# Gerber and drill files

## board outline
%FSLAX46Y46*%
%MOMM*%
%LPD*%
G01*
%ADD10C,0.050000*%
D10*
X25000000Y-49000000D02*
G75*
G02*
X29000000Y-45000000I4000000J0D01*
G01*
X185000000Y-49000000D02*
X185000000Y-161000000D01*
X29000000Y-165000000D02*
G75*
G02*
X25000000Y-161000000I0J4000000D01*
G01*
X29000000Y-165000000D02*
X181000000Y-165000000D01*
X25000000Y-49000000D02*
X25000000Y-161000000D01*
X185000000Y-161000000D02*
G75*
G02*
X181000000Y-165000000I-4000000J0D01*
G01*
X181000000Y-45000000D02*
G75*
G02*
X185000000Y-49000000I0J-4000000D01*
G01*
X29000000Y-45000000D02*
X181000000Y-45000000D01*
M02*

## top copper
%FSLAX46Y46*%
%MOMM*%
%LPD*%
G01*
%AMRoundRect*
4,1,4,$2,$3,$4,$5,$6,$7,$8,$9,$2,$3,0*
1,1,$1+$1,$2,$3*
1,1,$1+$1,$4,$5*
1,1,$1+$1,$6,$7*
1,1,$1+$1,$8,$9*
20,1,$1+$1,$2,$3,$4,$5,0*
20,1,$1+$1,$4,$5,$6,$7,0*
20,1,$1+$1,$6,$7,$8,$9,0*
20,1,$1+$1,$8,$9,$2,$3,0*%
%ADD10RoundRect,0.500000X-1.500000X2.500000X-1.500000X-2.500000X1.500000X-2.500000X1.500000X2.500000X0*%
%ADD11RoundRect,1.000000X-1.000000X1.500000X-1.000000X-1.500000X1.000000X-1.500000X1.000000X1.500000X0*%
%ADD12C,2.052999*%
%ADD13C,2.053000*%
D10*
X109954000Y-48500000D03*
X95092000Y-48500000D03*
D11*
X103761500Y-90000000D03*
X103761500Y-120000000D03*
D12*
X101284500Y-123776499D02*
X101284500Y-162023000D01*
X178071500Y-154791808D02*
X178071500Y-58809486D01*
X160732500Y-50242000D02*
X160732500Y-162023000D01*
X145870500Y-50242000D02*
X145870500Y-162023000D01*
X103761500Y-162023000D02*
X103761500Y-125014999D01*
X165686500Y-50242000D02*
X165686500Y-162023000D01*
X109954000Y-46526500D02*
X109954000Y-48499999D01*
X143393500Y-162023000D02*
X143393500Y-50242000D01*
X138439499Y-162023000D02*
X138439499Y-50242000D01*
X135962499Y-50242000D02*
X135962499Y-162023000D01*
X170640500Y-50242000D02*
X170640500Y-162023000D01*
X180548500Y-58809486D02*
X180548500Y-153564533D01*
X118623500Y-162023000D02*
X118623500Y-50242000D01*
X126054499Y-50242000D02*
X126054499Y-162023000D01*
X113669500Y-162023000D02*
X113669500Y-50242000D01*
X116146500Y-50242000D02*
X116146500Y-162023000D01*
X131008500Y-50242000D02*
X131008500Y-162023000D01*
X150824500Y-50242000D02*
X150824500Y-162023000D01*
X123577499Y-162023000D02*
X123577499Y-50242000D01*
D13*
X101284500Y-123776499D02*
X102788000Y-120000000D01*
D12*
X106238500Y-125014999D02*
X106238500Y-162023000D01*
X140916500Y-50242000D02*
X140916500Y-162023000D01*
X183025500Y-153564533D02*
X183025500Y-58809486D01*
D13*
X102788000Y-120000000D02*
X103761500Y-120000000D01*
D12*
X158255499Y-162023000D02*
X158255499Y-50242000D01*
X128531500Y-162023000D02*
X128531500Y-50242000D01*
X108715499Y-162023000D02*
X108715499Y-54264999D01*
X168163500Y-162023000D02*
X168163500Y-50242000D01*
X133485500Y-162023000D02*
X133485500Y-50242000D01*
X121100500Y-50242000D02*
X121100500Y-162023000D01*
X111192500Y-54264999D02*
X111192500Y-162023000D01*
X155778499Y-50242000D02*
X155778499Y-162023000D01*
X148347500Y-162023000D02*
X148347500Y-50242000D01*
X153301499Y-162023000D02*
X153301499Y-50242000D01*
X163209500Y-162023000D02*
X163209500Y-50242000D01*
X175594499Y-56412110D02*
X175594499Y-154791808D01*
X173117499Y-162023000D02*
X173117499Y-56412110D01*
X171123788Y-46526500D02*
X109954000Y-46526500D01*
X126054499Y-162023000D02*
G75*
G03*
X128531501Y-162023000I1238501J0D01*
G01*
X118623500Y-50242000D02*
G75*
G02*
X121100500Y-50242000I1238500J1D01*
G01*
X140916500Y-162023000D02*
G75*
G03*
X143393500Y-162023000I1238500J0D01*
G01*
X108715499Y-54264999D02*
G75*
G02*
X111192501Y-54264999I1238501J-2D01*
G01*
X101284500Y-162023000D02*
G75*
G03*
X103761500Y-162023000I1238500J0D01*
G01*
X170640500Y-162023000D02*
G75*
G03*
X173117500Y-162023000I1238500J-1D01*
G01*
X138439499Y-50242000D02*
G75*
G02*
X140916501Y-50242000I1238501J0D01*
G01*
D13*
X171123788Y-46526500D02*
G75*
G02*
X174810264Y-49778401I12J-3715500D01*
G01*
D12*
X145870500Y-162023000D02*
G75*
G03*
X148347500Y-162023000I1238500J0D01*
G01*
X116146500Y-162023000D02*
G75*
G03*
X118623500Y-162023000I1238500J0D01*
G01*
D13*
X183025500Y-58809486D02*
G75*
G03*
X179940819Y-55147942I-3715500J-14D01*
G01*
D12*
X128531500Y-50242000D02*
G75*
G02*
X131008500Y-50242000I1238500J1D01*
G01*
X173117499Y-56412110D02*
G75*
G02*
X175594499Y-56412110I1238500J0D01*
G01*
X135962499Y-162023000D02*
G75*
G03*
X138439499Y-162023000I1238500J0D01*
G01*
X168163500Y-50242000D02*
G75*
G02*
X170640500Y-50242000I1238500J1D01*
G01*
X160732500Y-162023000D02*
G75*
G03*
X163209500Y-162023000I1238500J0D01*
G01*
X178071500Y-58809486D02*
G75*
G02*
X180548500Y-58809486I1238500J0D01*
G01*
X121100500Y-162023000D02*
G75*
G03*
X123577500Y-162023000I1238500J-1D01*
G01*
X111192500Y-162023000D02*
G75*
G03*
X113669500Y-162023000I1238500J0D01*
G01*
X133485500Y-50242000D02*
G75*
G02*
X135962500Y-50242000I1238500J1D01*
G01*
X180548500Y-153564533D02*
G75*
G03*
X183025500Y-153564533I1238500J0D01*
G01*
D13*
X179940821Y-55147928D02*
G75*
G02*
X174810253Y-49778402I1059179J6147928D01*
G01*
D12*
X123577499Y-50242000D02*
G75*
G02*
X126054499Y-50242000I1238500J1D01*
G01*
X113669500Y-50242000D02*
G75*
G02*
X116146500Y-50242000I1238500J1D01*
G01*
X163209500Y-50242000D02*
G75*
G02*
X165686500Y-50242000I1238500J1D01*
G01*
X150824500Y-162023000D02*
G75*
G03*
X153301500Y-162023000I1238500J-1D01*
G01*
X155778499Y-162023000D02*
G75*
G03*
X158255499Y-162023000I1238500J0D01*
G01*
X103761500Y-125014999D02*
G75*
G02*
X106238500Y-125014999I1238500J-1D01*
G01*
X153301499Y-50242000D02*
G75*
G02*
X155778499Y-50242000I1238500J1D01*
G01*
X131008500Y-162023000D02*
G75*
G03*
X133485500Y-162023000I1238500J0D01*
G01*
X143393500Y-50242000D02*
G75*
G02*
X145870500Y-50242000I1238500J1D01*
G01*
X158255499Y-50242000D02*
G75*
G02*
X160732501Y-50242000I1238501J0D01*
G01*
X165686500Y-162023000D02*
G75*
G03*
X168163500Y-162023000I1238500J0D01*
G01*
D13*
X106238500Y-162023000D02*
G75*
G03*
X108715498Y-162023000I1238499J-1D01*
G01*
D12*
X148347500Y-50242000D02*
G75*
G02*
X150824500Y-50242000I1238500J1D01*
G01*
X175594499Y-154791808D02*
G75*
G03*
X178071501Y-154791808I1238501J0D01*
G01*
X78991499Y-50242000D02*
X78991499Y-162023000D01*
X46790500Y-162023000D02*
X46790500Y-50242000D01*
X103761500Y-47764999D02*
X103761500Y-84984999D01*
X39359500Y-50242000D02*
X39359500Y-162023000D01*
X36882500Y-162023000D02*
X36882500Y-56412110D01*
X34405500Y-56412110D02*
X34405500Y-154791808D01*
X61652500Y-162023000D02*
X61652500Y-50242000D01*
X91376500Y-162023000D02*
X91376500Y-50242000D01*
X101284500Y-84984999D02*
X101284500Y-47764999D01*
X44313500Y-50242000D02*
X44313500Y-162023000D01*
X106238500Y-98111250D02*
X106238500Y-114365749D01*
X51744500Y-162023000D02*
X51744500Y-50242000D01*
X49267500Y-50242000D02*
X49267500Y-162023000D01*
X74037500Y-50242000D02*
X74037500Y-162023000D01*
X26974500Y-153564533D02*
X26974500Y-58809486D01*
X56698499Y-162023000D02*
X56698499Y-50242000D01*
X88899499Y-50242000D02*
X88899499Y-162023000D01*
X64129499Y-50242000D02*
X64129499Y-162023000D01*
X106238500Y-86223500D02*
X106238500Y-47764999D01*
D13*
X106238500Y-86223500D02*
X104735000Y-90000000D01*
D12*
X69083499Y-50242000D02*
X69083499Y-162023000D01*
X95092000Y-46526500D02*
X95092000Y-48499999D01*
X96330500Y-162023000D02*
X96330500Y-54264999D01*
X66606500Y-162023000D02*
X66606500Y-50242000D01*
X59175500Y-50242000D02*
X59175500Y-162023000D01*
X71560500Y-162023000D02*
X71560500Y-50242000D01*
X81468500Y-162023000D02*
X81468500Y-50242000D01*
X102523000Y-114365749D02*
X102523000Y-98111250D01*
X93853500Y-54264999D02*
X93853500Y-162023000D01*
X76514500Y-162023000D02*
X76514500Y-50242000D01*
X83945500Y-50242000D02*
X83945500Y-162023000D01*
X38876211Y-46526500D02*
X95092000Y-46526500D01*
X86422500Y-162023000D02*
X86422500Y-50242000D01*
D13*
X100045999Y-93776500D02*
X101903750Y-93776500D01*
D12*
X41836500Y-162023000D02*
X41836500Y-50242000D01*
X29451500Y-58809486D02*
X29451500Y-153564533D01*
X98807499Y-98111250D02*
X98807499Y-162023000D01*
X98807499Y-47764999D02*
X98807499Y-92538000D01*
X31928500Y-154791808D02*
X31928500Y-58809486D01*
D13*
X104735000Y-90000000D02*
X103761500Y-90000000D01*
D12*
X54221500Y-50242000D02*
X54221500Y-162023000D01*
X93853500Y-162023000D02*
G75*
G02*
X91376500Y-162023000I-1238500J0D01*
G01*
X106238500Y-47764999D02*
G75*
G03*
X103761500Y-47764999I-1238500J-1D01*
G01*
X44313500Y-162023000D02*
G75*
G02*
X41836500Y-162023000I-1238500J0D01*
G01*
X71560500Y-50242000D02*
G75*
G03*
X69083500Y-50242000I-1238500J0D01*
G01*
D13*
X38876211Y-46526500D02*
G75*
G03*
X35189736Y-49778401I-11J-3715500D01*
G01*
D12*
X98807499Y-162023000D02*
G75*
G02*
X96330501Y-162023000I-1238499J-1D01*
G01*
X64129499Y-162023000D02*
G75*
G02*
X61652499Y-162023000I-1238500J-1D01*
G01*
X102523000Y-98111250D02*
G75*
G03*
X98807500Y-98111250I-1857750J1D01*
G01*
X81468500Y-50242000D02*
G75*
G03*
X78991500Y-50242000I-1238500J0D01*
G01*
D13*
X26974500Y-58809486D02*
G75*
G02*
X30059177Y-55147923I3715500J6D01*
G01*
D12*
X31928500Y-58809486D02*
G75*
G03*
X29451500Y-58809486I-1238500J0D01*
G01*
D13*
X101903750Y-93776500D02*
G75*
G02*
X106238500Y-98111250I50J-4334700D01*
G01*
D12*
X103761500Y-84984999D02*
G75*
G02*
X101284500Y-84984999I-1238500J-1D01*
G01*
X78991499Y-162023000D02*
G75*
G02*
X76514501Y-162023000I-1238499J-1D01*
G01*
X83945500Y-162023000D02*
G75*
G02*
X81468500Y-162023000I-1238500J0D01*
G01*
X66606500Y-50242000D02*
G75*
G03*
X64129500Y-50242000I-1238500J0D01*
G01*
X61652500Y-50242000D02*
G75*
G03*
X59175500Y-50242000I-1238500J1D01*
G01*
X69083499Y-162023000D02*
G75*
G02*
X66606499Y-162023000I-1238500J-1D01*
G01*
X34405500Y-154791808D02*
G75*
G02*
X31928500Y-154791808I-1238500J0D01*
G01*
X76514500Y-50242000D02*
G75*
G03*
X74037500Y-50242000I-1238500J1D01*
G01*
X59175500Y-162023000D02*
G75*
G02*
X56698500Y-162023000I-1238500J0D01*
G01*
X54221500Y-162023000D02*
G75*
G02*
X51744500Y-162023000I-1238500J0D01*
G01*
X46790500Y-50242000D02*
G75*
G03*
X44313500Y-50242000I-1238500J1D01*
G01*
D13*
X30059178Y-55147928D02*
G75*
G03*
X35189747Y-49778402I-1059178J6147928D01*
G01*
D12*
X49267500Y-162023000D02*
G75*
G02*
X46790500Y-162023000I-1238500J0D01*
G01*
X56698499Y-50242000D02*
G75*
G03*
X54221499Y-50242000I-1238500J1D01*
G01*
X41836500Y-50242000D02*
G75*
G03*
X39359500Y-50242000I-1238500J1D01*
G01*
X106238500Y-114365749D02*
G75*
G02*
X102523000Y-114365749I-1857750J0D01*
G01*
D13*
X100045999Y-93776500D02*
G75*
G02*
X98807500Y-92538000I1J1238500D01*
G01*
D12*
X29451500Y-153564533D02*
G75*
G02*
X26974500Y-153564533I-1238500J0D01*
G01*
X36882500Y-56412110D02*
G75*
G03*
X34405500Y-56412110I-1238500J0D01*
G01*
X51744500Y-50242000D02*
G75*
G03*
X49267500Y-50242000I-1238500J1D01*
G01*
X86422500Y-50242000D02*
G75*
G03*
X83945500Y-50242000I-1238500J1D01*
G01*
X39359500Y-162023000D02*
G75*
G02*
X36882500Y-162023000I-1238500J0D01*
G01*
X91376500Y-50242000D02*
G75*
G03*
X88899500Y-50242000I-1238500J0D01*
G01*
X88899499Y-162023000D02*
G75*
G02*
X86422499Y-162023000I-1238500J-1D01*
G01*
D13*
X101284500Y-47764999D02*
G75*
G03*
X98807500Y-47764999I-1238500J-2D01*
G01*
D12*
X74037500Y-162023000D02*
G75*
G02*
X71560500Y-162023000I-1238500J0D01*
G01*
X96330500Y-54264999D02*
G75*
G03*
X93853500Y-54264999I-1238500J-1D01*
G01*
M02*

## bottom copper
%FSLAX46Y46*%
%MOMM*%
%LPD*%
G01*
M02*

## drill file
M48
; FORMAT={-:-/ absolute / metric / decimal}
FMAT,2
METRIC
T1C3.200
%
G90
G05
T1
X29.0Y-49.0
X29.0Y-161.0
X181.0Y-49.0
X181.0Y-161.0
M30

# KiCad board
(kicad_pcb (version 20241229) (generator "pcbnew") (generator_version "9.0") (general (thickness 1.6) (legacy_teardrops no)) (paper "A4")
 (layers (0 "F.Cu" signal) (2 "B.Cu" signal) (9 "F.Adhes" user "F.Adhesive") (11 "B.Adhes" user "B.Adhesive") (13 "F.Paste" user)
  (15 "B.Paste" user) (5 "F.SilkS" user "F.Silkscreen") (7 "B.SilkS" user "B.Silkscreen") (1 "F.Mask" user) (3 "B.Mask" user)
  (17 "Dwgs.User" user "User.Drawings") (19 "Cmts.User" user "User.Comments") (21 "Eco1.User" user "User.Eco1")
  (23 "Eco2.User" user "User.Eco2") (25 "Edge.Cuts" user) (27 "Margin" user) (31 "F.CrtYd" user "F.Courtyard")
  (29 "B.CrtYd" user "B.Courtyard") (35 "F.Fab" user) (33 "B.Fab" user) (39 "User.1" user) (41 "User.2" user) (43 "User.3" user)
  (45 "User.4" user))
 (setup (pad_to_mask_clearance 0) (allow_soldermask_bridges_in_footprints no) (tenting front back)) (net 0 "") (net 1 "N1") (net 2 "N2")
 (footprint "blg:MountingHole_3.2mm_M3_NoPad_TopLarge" (layer "F.Cu") (at 181 49)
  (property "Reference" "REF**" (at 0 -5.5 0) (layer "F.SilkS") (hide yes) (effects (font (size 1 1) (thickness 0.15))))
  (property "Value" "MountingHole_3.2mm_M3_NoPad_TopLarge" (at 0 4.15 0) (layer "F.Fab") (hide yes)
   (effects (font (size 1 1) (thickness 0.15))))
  (pad "" np_thru_hole circle (at 0 0) (size 7.6 7.6) (drill 3.2) (layers) (zone_connect 2)))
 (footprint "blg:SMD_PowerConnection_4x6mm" (layer "F.Cu") (at 109.954 48.5 -90)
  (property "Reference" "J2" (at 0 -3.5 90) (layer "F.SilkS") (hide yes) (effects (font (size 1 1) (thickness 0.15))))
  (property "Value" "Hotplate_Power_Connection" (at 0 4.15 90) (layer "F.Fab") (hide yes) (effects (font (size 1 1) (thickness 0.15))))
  (pad "1" smd roundrect (at 0 0 270) (size 6 4) (layers "F.Cu" "F.Mask" "F.Paste") (roundrect_rratio 0.125) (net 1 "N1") (zone_connect 2)))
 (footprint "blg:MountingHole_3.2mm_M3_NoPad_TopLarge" (layer "F.Cu") (at 29 161)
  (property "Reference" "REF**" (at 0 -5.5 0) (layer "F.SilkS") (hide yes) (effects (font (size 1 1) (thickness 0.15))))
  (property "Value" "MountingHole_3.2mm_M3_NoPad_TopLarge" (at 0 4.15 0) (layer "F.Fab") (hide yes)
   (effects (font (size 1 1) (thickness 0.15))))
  (pad "" np_thru_hole circle (at 0 0) (size 7.6 7.6) (drill 3.2) (layers) (zone_connect 2)))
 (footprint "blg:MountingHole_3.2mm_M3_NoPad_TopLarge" (layer "F.Cu") (at 181 161)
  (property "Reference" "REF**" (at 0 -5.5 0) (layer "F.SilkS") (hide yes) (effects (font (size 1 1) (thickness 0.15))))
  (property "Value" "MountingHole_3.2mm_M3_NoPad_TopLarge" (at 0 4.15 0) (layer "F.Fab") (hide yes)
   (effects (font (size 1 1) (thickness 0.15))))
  (pad "" np_thru_hole circle (at 0 0) (size 7.6 7.6) (drill 3.2) (layers) (zone_connect 2)))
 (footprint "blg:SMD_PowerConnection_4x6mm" (layer "F.Cu") (at 95.092 48.5 -90)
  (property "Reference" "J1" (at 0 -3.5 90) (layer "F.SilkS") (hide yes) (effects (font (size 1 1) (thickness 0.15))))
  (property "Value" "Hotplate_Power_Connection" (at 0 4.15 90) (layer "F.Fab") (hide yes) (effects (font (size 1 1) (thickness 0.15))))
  (pad "1" smd roundrect (at 0 0 270) (size 6 4) (layers "F.Cu" "F.Mask" "F.Paste") (roundrect_rratio 0.125) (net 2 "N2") (zone_connect 2)))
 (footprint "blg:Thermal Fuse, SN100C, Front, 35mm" (layer "F.Cu") (at 103.7615 105 -90)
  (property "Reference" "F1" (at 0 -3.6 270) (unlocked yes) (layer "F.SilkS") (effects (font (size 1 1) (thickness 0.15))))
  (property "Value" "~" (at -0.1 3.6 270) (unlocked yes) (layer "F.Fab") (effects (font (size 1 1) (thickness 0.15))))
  (pad "1" smd roundrect (at -15 0 270) (size 5 4) (layers "F.Cu" "F.Mask") (roundrect_rratio 0.25) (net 2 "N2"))
  (pad "2" smd roundrect (at 15 0 270) (size 5 4) (layers "F.Cu" "F.Mask") (roundrect_rratio 0.25) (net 1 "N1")))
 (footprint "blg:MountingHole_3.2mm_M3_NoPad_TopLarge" (layer "F.Cu") (at 29 49)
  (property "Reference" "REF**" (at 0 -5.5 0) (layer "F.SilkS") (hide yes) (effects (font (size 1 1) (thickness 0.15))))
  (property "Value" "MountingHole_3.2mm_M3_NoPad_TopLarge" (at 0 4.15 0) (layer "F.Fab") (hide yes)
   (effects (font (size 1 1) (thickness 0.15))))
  (pad "" np_thru_hole circle (at 0 0) (size 7.6 7.6) (drill 3.2) (layers) (zone_connect 2)))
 (gr_arc (start 25 49) (mid 26.171573 46.171573) (end 29 45) (stroke (width 0.05) (type solid)) (layer "Edge.Cuts"))
 (gr_line (start 185 49) (end 185 161) (stroke (width 0.05) (type default)) (layer "Edge.Cuts"))
 (gr_arc (start 29 165) (mid 26.171573 163.828427) (end 25 161) (stroke (width 0.05) (type solid)) (layer "Edge.Cuts"))
 (gr_line (start 29 165) (end 181 165) (stroke (width 0.05) (type default)) (layer "Edge.Cuts"))
 (gr_line (start 25 49) (end 25 161) (stroke (width 0.05) (type default)) (layer "Edge.Cuts"))
 (gr_arc (start 185 161) (mid 183.828427 163.828427) (end 181 165) (stroke (width 0.05) (type solid)) (layer "Edge.Cuts"))
 (gr_arc (start 181 45) (mid 183.828427 46.171573) (end 185 49) (stroke (width 0.05) (type solid)) (layer "Edge.Cuts"))
 (gr_line (start 29 45) (end 181 45) (stroke (width 0.05) (type default)) (layer "Edge.Cuts"))
 (segment (start 101.2845 123.776499) (end 101.2845 162.023) (width 2.052999) (layer "F.Cu") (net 1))
 (segment (start 178.0715 154.791808) (end 178.0715 58.809486) (width 2.052999) (layer "F.Cu") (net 1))
 (segment (start 160.7325 50.242) (end 160.7325 162.023) (width 2.052999) (layer "F.Cu") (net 1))
 (segment (start 145.8705 50.242) (end 145.8705 162.023) (width 2.052999) (layer "F.Cu") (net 1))
 (segment (start 103.7615 162.023) (end 103.7615 125.014999) (width 2.052999) (layer "F.Cu") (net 1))
 (segment (start 165.6865 50.242) (end 165.6865 162.023) (width 2.052999) (layer "F.Cu") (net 1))
 (segment (start 109.954 46.5265) (end 109.954 48.499999) (width 2.052999) (layer "F.Cu") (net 1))
 (segment (start 143.3935 162.023) (end 143.3935 50.242) (width 2.052999) (layer "F.Cu") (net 1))
 (segment (start 138.439499 162.023) (end 138.439499 50.242) (width 2.052999) (layer "F.Cu") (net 1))
 (segment (start 135.962499 50.242) (end 135.962499 162.023) (width 2.052999) (layer "F.Cu") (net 1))
 (segment (start 170.6405 50.242) (end 170.6405 162.023) (width 2.052999) (layer "F.Cu") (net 1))
 (segment (start 180.5485 58.809486) (end 180.5485 153.564533) (width 2.052999) (layer "F.Cu") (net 1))
 (segment (start 118.6235 162.023) (end 118.6235 50.242) (width 2.052999) (layer "F.Cu") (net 1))
 (segment (start 126.054499 50.242) (end 126.054499 162.023) (width 2.052999) (layer "F.Cu") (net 1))
 (segment (start 113.6695 162.023) (end 113.6695 50.242) (width 2.052999) (layer "F.Cu") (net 1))
 (segment (start 116.1465 50.242) (end 116.1465 162.023) (width 2.052999) (layer "F.Cu") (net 1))
 (segment (start 131.0085 50.242) (end 131.0085 162.023) (width 2.052999) (layer "F.Cu") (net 1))
 (segment (start 150.8245 50.242) (end 150.8245 162.023) (width 2.052999) (layer "F.Cu") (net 1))
 (segment (start 123.577499 162.023) (end 123.577499 50.242) (width 2.052999) (layer "F.Cu") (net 1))
 (segment (start 101.2845 123.776499) (end 102.788 120) (width 2.053) (layer "F.Cu") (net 1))
 (segment (start 106.2385 125.014999) (end 106.2385 162.023) (width 2.052999) (layer "F.Cu") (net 1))
 (segment (start 140.9165 50.242) (end 140.9165 162.023) (width 2.052999) (layer "F.Cu") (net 1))
 (segment (start 183.0255 153.564533) (end 183.0255 58.809486) (width 2.052999) (layer "F.Cu") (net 1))
 (segment (start 102.788 120) (end 103.7615 120) (width 2.053) (layer "F.Cu") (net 1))
 (segment (start 158.255499 162.023) (end 158.255499 50.242) (width 2.052999) (layer "F.Cu") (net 1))
 (segment (start 128.5315 162.023) (end 128.5315 50.242) (width 2.052999) (layer "F.Cu") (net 1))
 (segment (start 108.715499 162.023) (end 108.715499 54.264999) (width 2.052999) (layer "F.Cu") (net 1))
 (segment (start 168.1635 162.023) (end 168.1635 50.242) (width 2.052999) (layer "F.Cu") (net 1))
 (segment (start 133.4855 162.023) (end 133.4855 50.242) (width 2.052999) (layer "F.Cu") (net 1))
 (segment (start 121.1005 50.242) (end 121.1005 162.023) (width 2.052999) (layer "F.Cu") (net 1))
 (segment (start 111.1925 54.264999) (end 111.1925 162.023) (width 2.052999) (layer "F.Cu") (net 1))
 (segment (start 155.778499 50.242) (end 155.778499 162.023) (width 2.052999) (layer "F.Cu") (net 1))
 (segment (start 148.3475 162.023) (end 148.3475 50.242) (width 2.052999) (layer "F.Cu") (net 1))
 (segment (start 153.301499 162.023) (end 153.301499 50.242) (width 2.052999) (layer "F.Cu") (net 1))
 (segment (start 163.2095 162.023) (end 163.2095 50.242) (width 2.052999) (layer "F.Cu") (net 1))
 (segment (start 175.594499 56.41211) (end 175.594499 154.791808) (width 2.052999) (layer "F.Cu") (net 1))
 (segment (start 173.117499 162.023) (end 173.117499 56.41211) (width 2.052999) (layer "F.Cu") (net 1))
 (segment (start 171.123788 46.5265) (end 109.954 46.5265) (width 2.052999) (layer "F.Cu") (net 1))
 (arc (start 126.054499 162.023) (mid 127.292999 163.2615) (end 128.5315 162.023) (width 2.052999) (layer "F.Cu") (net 1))
 (arc (start 118.6235 50.242) (mid 119.862 49.003499) (end 121.1005 50.242) (width 2.052999) (layer "F.Cu") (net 1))
 (arc (start 140.9165 162.023) (mid 142.155 163.2615) (end 143.3935 162.023) (width 2.052999) (layer "F.Cu") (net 1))
 (arc (start 108.715499 54.264999) (mid 109.954 53.0265) (end 111.1925 54.264999) (width 2.052999) (layer "F.Cu") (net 1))
 (arc (start 101.2845 162.023) (mid 102.523 163.2615) (end 103.7615 162.023) (width 2.052999) (layer "F.Cu") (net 1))
 (arc (start 170.6405 162.023) (mid 171.879 163.2615) (end 173.117499 162.023) (width 2.052999) (layer "F.Cu") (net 1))
 (arc (start 138.439499 50.242) (mid 139.678 49.003499) (end 140.9165 50.242) (width 2.052999) (layer "F.Cu") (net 1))
 (arc (start 171.123788 46.5265) (mid 173.581678 47.455654) (end 174.810252 49.778402) (width 2.053) (layer "F.Cu") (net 1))
 (arc (start 145.8705 162.023) (mid 147.108999 163.2615) (end 148.3475 162.023) (width 2.052999) (layer "F.Cu") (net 1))
 (arc (start 116.1465 162.023) (mid 117.384999 163.2615) (end 118.6235 162.023) (width 2.052999) (layer "F.Cu") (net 1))
 (arc (start 183.0255 58.809486) (mid 181.907622 56.152928) (end 179.940821 55.147928) (width 2.053) (layer "F.Cu") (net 1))
 (arc (start 128.5315 50.242) (mid 129.77 49.003499) (end 131.0085 50.242) (width 2.052999) (layer "F.Cu") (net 1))
 (arc (start 173.117499 56.41211) (mid 174.356 55.17361) (end 175.594499 56.41211) (width 2.052999) (layer "F.Cu") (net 1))
 (arc (start 135.962499 162.023) (mid 137.201 163.2615) (end 138.439499 162.023) (width 2.052999) (layer "F.Cu") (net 1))
 (arc (start 168.1635 50.242) (mid 169.402 49.003499) (end 170.6405 50.242) (width 2.052999) (layer "F.Cu") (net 1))
 (arc (start 160.7325 162.023) (mid 161.971 163.2615) (end 163.2095 162.023) (width 2.052999) (layer "F.Cu") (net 1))
 (arc (start 178.0715 58.809486) (mid 179.31 57.570986) (end 180.5485 58.809486) (width 2.052999) (layer "F.Cu") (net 1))
 (arc (start 121.1005 162.023) (mid 122.338999 163.2615) (end 123.577499 162.023) (width 2.052999) (layer "F.Cu") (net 1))
 (arc (start 111.1925 162.023) (mid 112.430999 163.2615) (end 113.6695 162.023) (width 2.052999) (layer "F.Cu") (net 1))
 (arc (start 133.4855 50.242) (mid 134.724 49.003499) (end 135.962499 50.242) (width 2.052999) (layer "F.Cu") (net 1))
 (arc (start 180.5485 153.564533) (mid 181.787 154.803033) (end 183.0255 153.564533) (width 2.052999) (layer "F.Cu") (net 1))
 (arc (start 179.940821 55.147928) (mid 176.489491 53.309779) (end 174.810252 49.778402) (width 2.053) (layer "F.Cu") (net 1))
 (arc (start 123.577499 50.242) (mid 124.816 49.003499) (end 126.054499 50.242) (width 2.052999) (layer "F.Cu") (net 1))
 (arc (start 113.6695 50.242) (mid 114.908 49.003499) (end 116.1465 50.242) (width 2.052999) (layer "F.Cu") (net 1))
 (arc (start 163.2095 50.242) (mid 164.447999 49.003499) (end 165.6865 50.242) (width 2.052999) (layer "F.Cu") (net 1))
 (arc (start 150.8245 162.023) (mid 152.063 163.2615) (end 153.301499 162.023) (width 2.052999) (layer "F.Cu") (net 1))
 (arc (start 155.778499 162.023) (mid 157.017 163.2615) (end 158.255499 162.023) (width 2.052999) (layer "F.Cu") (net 1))
 (arc (start 103.7615 125.014999) (mid 105 123.7765) (end 106.2385 125.014999) (width 2.052999) (layer "F.Cu") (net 1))
 (arc (start 153.301499 50.242) (mid 154.54 49.003499) (end 155.778499 50.242) (width 2.052999) (layer "F.Cu") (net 1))
 (arc (start 131.0085 162.023) (mid 132.247 163.2615) (end 133.4855 162.023) (width 2.052999) (layer "F.Cu") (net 1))
 (arc (start 143.3935 50.242) (mid 144.631999 49.003499) (end 145.8705 50.242) (width 2.052999) (layer "F.Cu") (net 1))
 (arc (start 158.255499 50.242) (mid 159.494 49.003499) (end 160.7325 50.242) (width 2.052999) (layer "F.Cu") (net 1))
 (arc (start 165.6865 162.023) (mid 166.924999 163.2615) (end 168.1635 162.023) (width 2.052999) (layer "F.Cu") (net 1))
 (arc (start 106.2385 162.023) (mid 107.477 163.2615) (end 108.715499 162.023) (width 2.053) (layer "F.Cu") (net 1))
 (arc (start 148.3475 50.242) (mid 149.585999 49.003499) (end 150.8245 50.242) (width 2.052999) (layer "F.Cu") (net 1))
 (arc (start 175.594499 154.791808) (mid 176.833 156.030308) (end 178.0715 154.791808) (width 2.052999) (layer "F.Cu") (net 1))
 (segment (start 78.991499 50.242) (end 78.991499 162.023) (width 2.052999) (layer "F.Cu") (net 2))
 (segment (start 46.7905 162.023) (end 46.7905 50.242) (width 2.052999) (layer "F.Cu") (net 2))
 (segment (start 103.7615 47.764999) (end 103.7615 84.984999) (width 2.052999) (layer "F.Cu") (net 2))
 (segment (start 39.3595 50.242) (end 39.3595 162.023) (width 2.052999) (layer "F.Cu") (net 2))
 (segment (start 36.8825 162.023) (end 36.8825 56.41211) (width 2.052999) (layer "F.Cu") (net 2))
 (segment (start 34.4055 56.41211) (end 34.4055 154.791808) (width 2.052999) (layer "F.Cu") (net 2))
 (segment (start 61.6525 162.023) (end 61.6525 50.242) (width 2.052999) (layer "F.Cu") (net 2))
 (segment (start 91.3765 162.023) (end 91.3765 50.242) (width 2.052999) (layer "F.Cu") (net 2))
 (segment (start 101.2845 84.984999) (end 101.2845 47.764999) (width 2.052999) (layer "F.Cu") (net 2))
 (segment (start 44.3135 50.242) (end 44.3135 162.023) (width 2.052999) (layer "F.Cu") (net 2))
 (segment (start 106.2385 98.11125) (end 106.2385 114.365749) (width 2.052999) (layer "F.Cu") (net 2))
 (segment (start 51.7445 162.023) (end 51.7445 50.242) (width 2.052999) (layer "F.Cu") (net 2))
 (segment (start 49.2675 50.242) (end 49.2675 162.023) (width 2.052999) (layer "F.Cu") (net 2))
 (segment (start 74.0375 50.242) (end 74.0375 162.023) (width 2.052999) (layer "F.Cu") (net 2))
 (segment (start 26.9745 153.564533) (end 26.9745 58.809486) (width 2.052999) (layer "F.Cu") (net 2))
 (segment (start 56.698499 162.023) (end 56.698499 50.242) (width 2.052999) (layer "F.Cu") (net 2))
 (segment (start 88.899499 50.242) (end 88.899499 162.023) (width 2.052999) (layer "F.Cu") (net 2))
 (segment (start 64.129499 50.242) (end 64.129499 162.023) (width 2.052999) (layer "F.Cu") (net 2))
 (segment (start 106.2385 86.2235) (end 106.2385 47.764999) (width 2.052999) (layer "F.Cu") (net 2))
 (segment (start 106.2385 86.2235) (end 104.735 90) (width 2.053) (layer "F.Cu") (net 2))
 (segment (start 69.083499 50.242) (end 69.083499 162.023) (width 2.052999) (layer "F.Cu") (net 2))
 (segment (start 95.092 46.5265) (end 95.092 48.499999) (width 2.052999) (layer "F.Cu") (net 2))
 (segment (start 96.3305 162.023) (end 96.3305 54.264999) (width 2.052999) (layer "F.Cu") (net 2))
 (segment (start 66.6065 162.023) (end 66.6065 50.242) (width 2.052999) (layer "F.Cu") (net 2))
 (segment (start 59.1755 50.242) (end 59.1755 162.023) (width 2.052999) (layer "F.Cu") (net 2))
 (segment (start 71.5605 162.023) (end 71.5605 50.242) (width 2.052999) (layer "F.Cu") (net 2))
 (segment (start 81.4685 162.023) (end 81.4685 50.242) (width 2.052999) (layer "F.Cu") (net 2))
 (segment (start 102.523 114.365749) (end 102.523 98.11125) (width 2.052999) (layer "F.Cu") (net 2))
 (segment (start 93.8535 54.264999) (end 93.8535 162.023) (width 2.052999) (layer "F.Cu") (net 2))
 (segment (start 76.5145 162.023) (end 76.5145 50.242) (width 2.052999) (layer "F.Cu") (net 2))
 (segment (start 83.9455 50.242) (end 83.9455 162.023) (width 2.052999) (layer "F.Cu") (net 2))
 (segment (start 38.876211 46.5265) (end 95.092 46.5265) (width 2.052999) (layer "F.Cu") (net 2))
 (segment (start 86.4225 162.023) (end 86.4225 50.242) (width 2.052999) (layer "F.Cu") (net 2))
 (segment (start 100.045999 93.7765) (end 101.90375 93.7765) (width 2.053) (layer "F.Cu") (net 2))
 (segment (start 41.8365 162.023) (end 41.8365 50.242) (width 2.052999) (layer "F.Cu") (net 2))
 (segment (start 29.4515 58.809486) (end 29.4515 153.564533) (width 2.052999) (layer "F.Cu") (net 2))
 (segment (start 98.807499 98.11125) (end 98.807499 162.023) (width 2.052999) (layer "F.Cu") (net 2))
 (segment (start 98.807499 47.764999) (end 98.807499 92.538) (width 2.052999) (layer "F.Cu") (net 2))
 (segment (start 31.9285 154.791808) (end 31.9285 58.809486) (width 2.052999) (layer "F.Cu") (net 2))
 (segment (start 104.735 90) (end 103.7615 90) (width 2.053) (layer "F.Cu") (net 2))
 (segment (start 54.2215 50.242) (end 54.2215 162.023) (width 2.052999) (layer "F.Cu") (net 2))
 (arc (start 93.8535 162.023) (mid 92.615 163.2615) (end 91.3765 162.023) (width 2.052999) (layer "F.Cu") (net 2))
 (arc (start 106.2385 47.764999) (mid 105 46.5265) (end 103.7615 47.764999) (width 2.052999) (layer "F.Cu") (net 2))
 (arc (start 44.3135 162.023) (mid 43.074999 163.2615) (end 41.8365 162.023) (width 2.052999) (layer "F.Cu") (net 2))
 (arc (start 71.5605 50.242) (mid 70.322 49.003499) (end 69.083499 50.242) (width 2.052999) (layer "F.Cu") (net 2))
 (arc (start 38.876211 46.5265) (mid 36.418321 47.455654) (end 35.189747 49.778402) (width 2.053) (layer "F.Cu") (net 2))
 (arc (start 98.807499 162.023) (mid 97.568999 163.2615) (end 96.3305 162.023) (width 2.052999) (layer "F.Cu") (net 2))
 (arc (start 64.129499 162.023) (mid 62.891 163.2615) (end 61.6525 162.023) (width 2.052999) (layer "F.Cu") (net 2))
 (arc (start 102.523 98.11125) (mid 100.66525 96.253499) (end 98.807499 98.11125) (width 2.052999) (layer "F.Cu") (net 2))
 (arc (start 81.4685 50.242) (mid 80.229999 49.003499) (end 78.991499 50.242) (width 2.052999) (layer "F.Cu") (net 2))
 (arc (start 26.9745 58.809486) (mid 28.092377 56.152928) (end 30.059178 55.147928) (width 2.053) (layer "F.Cu") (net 2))
 (arc (start 31.9285 58.809486) (mid 30.689999 57.570986) (end 29.4515 58.809486) (width 2.052999) (layer "F.Cu") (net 2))
 (arc (start 101.90375 93.7765) (mid 104.968881 95.046118) (end 106.2385 98.11125) (width 2.053) (layer "F.Cu") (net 2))
 (arc (start 103.7615 84.984999) (mid 102.523 86.2235) (end 101.2845 84.984999) (width 2.052999) (layer "F.Cu") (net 2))
 (arc (start 78.991499 162.023) (mid 77.753 163.2615) (end 76.5145 162.023) (width 2.052999) (layer "F.Cu") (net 2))
 (arc (start 83.9455 162.023) (mid 82.707 163.2615) (end 81.4685 162.023) (width 2.052999) (layer "F.Cu") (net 2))
 (arc (start 66.6065 50.242) (mid 65.367999 49.003499) (end 64.129499 50.242) (width 2.052999) (layer "F.Cu") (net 2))
 (arc (start 61.6525 50.242) (mid 60.413999 49.003499) (end 59.1755 50.242) (width 2.052999) (layer "F.Cu") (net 2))
 (arc (start 69.083499 162.023) (mid 67.845 163.2615) (end 66.6065 162.023) (width 2.052999) (layer "F.Cu") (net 2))
 (arc (start 34.4055 154.791808) (mid 33.166999 156.030308) (end 31.9285 154.791808) (width 2.052999) (layer "F.Cu") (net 2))
 (arc (start 76.5145 50.242) (mid 75.276 49.003499) (end 74.0375 50.242) (width 2.052999) (layer "F.Cu") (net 2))
 (arc (start 59.1755 162.023) (mid 57.937 163.2615) (end 56.698499 162.023) (width 2.052999) (layer "F.Cu") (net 2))
 (arc (start 54.2215 162.023) (mid 52.983 163.2615) (end 51.7445 162.023) (width 2.052999) (layer "F.Cu") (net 2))
 (arc (start 46.7905 50.242) (mid 45.551999 49.003499) (end 44.3135 50.242) (width 2.052999) (layer "F.Cu") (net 2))
 (arc (start 30.059178 55.147928) (mid 33.510508 53.309779) (end 35.189747 49.778402) (width 2.053) (layer "F.Cu") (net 2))
 (arc (start 49.2675 162.023) (mid 48.029 163.2615) (end 46.7905 162.023) (width 2.052999) (layer "F.Cu") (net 2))
 (arc (start 56.698499 50.242) (mid 55.459999 49.003499) (end 54.2215 50.242) (width 2.052999) (layer "F.Cu") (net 2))
 (arc (start 41.8365 50.242) (mid 40.597999 49.003499) (end 39.3595 50.242) (width 2.052999) (layer "F.Cu") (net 2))
 (arc (start 106.2385 114.365749) (mid 104.380749 116.223499) (end 102.523 114.365749) (width 2.052999) (layer "F.Cu") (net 2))
 (arc (start 100.045999 93.7765) (mid 99.170248 93.413751) (end 98.807499 92.538) (width 2.053) (layer "F.Cu") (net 2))
 (arc (start 29.4515 153.564533) (mid 28.212999 154.803033) (end 26.9745 153.564533) (width 2.052999) (layer "F.Cu") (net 2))
 (arc (start 36.8825 56.41211) (mid 35.644 55.17361) (end 34.4055 56.41211) (width 2.052999) (layer "F.Cu") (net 2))
 (arc (start 51.7445 50.242) (mid 50.505999 49.003499) (end 49.2675 50.242) (width 2.052999) (layer "F.Cu") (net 2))
 (arc (start 86.4225 50.242) (mid 85.184 49.003499) (end 83.9455 50.242) (width 2.052999) (layer "F.Cu") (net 2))
 (arc (start 39.3595 162.023) (mid 38.120999 163.2615) (end 36.8825 162.023) (width 2.052999) (layer "F.Cu") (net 2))
 (arc (start 91.3765 50.242) (mid 90.137999 49.003499) (end 88.899499 50.242) (width 2.052999) (layer "F.Cu") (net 2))
 (arc (start 88.899499 162.023) (mid 87.661 163.2615) (end 86.4225 162.023) (width 2.052999) (layer "F.Cu") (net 2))
 (arc (start 101.2845 47.764999) (mid 100.045999 46.5265) (end 98.807499 47.764999) (width 2.053) (layer "F.Cu") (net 2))
 (arc (start 74.0375 162.023) (mid 72.799 163.2615) (end 71.5605 162.023) (width 2.052999) (layer "F.Cu") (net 2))
 (arc (start 96.3305 54.264999) (mid 95.092 53.0265) (end 93.8535 54.264999) (width 2.052999) (layer "F.Cu") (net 2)))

